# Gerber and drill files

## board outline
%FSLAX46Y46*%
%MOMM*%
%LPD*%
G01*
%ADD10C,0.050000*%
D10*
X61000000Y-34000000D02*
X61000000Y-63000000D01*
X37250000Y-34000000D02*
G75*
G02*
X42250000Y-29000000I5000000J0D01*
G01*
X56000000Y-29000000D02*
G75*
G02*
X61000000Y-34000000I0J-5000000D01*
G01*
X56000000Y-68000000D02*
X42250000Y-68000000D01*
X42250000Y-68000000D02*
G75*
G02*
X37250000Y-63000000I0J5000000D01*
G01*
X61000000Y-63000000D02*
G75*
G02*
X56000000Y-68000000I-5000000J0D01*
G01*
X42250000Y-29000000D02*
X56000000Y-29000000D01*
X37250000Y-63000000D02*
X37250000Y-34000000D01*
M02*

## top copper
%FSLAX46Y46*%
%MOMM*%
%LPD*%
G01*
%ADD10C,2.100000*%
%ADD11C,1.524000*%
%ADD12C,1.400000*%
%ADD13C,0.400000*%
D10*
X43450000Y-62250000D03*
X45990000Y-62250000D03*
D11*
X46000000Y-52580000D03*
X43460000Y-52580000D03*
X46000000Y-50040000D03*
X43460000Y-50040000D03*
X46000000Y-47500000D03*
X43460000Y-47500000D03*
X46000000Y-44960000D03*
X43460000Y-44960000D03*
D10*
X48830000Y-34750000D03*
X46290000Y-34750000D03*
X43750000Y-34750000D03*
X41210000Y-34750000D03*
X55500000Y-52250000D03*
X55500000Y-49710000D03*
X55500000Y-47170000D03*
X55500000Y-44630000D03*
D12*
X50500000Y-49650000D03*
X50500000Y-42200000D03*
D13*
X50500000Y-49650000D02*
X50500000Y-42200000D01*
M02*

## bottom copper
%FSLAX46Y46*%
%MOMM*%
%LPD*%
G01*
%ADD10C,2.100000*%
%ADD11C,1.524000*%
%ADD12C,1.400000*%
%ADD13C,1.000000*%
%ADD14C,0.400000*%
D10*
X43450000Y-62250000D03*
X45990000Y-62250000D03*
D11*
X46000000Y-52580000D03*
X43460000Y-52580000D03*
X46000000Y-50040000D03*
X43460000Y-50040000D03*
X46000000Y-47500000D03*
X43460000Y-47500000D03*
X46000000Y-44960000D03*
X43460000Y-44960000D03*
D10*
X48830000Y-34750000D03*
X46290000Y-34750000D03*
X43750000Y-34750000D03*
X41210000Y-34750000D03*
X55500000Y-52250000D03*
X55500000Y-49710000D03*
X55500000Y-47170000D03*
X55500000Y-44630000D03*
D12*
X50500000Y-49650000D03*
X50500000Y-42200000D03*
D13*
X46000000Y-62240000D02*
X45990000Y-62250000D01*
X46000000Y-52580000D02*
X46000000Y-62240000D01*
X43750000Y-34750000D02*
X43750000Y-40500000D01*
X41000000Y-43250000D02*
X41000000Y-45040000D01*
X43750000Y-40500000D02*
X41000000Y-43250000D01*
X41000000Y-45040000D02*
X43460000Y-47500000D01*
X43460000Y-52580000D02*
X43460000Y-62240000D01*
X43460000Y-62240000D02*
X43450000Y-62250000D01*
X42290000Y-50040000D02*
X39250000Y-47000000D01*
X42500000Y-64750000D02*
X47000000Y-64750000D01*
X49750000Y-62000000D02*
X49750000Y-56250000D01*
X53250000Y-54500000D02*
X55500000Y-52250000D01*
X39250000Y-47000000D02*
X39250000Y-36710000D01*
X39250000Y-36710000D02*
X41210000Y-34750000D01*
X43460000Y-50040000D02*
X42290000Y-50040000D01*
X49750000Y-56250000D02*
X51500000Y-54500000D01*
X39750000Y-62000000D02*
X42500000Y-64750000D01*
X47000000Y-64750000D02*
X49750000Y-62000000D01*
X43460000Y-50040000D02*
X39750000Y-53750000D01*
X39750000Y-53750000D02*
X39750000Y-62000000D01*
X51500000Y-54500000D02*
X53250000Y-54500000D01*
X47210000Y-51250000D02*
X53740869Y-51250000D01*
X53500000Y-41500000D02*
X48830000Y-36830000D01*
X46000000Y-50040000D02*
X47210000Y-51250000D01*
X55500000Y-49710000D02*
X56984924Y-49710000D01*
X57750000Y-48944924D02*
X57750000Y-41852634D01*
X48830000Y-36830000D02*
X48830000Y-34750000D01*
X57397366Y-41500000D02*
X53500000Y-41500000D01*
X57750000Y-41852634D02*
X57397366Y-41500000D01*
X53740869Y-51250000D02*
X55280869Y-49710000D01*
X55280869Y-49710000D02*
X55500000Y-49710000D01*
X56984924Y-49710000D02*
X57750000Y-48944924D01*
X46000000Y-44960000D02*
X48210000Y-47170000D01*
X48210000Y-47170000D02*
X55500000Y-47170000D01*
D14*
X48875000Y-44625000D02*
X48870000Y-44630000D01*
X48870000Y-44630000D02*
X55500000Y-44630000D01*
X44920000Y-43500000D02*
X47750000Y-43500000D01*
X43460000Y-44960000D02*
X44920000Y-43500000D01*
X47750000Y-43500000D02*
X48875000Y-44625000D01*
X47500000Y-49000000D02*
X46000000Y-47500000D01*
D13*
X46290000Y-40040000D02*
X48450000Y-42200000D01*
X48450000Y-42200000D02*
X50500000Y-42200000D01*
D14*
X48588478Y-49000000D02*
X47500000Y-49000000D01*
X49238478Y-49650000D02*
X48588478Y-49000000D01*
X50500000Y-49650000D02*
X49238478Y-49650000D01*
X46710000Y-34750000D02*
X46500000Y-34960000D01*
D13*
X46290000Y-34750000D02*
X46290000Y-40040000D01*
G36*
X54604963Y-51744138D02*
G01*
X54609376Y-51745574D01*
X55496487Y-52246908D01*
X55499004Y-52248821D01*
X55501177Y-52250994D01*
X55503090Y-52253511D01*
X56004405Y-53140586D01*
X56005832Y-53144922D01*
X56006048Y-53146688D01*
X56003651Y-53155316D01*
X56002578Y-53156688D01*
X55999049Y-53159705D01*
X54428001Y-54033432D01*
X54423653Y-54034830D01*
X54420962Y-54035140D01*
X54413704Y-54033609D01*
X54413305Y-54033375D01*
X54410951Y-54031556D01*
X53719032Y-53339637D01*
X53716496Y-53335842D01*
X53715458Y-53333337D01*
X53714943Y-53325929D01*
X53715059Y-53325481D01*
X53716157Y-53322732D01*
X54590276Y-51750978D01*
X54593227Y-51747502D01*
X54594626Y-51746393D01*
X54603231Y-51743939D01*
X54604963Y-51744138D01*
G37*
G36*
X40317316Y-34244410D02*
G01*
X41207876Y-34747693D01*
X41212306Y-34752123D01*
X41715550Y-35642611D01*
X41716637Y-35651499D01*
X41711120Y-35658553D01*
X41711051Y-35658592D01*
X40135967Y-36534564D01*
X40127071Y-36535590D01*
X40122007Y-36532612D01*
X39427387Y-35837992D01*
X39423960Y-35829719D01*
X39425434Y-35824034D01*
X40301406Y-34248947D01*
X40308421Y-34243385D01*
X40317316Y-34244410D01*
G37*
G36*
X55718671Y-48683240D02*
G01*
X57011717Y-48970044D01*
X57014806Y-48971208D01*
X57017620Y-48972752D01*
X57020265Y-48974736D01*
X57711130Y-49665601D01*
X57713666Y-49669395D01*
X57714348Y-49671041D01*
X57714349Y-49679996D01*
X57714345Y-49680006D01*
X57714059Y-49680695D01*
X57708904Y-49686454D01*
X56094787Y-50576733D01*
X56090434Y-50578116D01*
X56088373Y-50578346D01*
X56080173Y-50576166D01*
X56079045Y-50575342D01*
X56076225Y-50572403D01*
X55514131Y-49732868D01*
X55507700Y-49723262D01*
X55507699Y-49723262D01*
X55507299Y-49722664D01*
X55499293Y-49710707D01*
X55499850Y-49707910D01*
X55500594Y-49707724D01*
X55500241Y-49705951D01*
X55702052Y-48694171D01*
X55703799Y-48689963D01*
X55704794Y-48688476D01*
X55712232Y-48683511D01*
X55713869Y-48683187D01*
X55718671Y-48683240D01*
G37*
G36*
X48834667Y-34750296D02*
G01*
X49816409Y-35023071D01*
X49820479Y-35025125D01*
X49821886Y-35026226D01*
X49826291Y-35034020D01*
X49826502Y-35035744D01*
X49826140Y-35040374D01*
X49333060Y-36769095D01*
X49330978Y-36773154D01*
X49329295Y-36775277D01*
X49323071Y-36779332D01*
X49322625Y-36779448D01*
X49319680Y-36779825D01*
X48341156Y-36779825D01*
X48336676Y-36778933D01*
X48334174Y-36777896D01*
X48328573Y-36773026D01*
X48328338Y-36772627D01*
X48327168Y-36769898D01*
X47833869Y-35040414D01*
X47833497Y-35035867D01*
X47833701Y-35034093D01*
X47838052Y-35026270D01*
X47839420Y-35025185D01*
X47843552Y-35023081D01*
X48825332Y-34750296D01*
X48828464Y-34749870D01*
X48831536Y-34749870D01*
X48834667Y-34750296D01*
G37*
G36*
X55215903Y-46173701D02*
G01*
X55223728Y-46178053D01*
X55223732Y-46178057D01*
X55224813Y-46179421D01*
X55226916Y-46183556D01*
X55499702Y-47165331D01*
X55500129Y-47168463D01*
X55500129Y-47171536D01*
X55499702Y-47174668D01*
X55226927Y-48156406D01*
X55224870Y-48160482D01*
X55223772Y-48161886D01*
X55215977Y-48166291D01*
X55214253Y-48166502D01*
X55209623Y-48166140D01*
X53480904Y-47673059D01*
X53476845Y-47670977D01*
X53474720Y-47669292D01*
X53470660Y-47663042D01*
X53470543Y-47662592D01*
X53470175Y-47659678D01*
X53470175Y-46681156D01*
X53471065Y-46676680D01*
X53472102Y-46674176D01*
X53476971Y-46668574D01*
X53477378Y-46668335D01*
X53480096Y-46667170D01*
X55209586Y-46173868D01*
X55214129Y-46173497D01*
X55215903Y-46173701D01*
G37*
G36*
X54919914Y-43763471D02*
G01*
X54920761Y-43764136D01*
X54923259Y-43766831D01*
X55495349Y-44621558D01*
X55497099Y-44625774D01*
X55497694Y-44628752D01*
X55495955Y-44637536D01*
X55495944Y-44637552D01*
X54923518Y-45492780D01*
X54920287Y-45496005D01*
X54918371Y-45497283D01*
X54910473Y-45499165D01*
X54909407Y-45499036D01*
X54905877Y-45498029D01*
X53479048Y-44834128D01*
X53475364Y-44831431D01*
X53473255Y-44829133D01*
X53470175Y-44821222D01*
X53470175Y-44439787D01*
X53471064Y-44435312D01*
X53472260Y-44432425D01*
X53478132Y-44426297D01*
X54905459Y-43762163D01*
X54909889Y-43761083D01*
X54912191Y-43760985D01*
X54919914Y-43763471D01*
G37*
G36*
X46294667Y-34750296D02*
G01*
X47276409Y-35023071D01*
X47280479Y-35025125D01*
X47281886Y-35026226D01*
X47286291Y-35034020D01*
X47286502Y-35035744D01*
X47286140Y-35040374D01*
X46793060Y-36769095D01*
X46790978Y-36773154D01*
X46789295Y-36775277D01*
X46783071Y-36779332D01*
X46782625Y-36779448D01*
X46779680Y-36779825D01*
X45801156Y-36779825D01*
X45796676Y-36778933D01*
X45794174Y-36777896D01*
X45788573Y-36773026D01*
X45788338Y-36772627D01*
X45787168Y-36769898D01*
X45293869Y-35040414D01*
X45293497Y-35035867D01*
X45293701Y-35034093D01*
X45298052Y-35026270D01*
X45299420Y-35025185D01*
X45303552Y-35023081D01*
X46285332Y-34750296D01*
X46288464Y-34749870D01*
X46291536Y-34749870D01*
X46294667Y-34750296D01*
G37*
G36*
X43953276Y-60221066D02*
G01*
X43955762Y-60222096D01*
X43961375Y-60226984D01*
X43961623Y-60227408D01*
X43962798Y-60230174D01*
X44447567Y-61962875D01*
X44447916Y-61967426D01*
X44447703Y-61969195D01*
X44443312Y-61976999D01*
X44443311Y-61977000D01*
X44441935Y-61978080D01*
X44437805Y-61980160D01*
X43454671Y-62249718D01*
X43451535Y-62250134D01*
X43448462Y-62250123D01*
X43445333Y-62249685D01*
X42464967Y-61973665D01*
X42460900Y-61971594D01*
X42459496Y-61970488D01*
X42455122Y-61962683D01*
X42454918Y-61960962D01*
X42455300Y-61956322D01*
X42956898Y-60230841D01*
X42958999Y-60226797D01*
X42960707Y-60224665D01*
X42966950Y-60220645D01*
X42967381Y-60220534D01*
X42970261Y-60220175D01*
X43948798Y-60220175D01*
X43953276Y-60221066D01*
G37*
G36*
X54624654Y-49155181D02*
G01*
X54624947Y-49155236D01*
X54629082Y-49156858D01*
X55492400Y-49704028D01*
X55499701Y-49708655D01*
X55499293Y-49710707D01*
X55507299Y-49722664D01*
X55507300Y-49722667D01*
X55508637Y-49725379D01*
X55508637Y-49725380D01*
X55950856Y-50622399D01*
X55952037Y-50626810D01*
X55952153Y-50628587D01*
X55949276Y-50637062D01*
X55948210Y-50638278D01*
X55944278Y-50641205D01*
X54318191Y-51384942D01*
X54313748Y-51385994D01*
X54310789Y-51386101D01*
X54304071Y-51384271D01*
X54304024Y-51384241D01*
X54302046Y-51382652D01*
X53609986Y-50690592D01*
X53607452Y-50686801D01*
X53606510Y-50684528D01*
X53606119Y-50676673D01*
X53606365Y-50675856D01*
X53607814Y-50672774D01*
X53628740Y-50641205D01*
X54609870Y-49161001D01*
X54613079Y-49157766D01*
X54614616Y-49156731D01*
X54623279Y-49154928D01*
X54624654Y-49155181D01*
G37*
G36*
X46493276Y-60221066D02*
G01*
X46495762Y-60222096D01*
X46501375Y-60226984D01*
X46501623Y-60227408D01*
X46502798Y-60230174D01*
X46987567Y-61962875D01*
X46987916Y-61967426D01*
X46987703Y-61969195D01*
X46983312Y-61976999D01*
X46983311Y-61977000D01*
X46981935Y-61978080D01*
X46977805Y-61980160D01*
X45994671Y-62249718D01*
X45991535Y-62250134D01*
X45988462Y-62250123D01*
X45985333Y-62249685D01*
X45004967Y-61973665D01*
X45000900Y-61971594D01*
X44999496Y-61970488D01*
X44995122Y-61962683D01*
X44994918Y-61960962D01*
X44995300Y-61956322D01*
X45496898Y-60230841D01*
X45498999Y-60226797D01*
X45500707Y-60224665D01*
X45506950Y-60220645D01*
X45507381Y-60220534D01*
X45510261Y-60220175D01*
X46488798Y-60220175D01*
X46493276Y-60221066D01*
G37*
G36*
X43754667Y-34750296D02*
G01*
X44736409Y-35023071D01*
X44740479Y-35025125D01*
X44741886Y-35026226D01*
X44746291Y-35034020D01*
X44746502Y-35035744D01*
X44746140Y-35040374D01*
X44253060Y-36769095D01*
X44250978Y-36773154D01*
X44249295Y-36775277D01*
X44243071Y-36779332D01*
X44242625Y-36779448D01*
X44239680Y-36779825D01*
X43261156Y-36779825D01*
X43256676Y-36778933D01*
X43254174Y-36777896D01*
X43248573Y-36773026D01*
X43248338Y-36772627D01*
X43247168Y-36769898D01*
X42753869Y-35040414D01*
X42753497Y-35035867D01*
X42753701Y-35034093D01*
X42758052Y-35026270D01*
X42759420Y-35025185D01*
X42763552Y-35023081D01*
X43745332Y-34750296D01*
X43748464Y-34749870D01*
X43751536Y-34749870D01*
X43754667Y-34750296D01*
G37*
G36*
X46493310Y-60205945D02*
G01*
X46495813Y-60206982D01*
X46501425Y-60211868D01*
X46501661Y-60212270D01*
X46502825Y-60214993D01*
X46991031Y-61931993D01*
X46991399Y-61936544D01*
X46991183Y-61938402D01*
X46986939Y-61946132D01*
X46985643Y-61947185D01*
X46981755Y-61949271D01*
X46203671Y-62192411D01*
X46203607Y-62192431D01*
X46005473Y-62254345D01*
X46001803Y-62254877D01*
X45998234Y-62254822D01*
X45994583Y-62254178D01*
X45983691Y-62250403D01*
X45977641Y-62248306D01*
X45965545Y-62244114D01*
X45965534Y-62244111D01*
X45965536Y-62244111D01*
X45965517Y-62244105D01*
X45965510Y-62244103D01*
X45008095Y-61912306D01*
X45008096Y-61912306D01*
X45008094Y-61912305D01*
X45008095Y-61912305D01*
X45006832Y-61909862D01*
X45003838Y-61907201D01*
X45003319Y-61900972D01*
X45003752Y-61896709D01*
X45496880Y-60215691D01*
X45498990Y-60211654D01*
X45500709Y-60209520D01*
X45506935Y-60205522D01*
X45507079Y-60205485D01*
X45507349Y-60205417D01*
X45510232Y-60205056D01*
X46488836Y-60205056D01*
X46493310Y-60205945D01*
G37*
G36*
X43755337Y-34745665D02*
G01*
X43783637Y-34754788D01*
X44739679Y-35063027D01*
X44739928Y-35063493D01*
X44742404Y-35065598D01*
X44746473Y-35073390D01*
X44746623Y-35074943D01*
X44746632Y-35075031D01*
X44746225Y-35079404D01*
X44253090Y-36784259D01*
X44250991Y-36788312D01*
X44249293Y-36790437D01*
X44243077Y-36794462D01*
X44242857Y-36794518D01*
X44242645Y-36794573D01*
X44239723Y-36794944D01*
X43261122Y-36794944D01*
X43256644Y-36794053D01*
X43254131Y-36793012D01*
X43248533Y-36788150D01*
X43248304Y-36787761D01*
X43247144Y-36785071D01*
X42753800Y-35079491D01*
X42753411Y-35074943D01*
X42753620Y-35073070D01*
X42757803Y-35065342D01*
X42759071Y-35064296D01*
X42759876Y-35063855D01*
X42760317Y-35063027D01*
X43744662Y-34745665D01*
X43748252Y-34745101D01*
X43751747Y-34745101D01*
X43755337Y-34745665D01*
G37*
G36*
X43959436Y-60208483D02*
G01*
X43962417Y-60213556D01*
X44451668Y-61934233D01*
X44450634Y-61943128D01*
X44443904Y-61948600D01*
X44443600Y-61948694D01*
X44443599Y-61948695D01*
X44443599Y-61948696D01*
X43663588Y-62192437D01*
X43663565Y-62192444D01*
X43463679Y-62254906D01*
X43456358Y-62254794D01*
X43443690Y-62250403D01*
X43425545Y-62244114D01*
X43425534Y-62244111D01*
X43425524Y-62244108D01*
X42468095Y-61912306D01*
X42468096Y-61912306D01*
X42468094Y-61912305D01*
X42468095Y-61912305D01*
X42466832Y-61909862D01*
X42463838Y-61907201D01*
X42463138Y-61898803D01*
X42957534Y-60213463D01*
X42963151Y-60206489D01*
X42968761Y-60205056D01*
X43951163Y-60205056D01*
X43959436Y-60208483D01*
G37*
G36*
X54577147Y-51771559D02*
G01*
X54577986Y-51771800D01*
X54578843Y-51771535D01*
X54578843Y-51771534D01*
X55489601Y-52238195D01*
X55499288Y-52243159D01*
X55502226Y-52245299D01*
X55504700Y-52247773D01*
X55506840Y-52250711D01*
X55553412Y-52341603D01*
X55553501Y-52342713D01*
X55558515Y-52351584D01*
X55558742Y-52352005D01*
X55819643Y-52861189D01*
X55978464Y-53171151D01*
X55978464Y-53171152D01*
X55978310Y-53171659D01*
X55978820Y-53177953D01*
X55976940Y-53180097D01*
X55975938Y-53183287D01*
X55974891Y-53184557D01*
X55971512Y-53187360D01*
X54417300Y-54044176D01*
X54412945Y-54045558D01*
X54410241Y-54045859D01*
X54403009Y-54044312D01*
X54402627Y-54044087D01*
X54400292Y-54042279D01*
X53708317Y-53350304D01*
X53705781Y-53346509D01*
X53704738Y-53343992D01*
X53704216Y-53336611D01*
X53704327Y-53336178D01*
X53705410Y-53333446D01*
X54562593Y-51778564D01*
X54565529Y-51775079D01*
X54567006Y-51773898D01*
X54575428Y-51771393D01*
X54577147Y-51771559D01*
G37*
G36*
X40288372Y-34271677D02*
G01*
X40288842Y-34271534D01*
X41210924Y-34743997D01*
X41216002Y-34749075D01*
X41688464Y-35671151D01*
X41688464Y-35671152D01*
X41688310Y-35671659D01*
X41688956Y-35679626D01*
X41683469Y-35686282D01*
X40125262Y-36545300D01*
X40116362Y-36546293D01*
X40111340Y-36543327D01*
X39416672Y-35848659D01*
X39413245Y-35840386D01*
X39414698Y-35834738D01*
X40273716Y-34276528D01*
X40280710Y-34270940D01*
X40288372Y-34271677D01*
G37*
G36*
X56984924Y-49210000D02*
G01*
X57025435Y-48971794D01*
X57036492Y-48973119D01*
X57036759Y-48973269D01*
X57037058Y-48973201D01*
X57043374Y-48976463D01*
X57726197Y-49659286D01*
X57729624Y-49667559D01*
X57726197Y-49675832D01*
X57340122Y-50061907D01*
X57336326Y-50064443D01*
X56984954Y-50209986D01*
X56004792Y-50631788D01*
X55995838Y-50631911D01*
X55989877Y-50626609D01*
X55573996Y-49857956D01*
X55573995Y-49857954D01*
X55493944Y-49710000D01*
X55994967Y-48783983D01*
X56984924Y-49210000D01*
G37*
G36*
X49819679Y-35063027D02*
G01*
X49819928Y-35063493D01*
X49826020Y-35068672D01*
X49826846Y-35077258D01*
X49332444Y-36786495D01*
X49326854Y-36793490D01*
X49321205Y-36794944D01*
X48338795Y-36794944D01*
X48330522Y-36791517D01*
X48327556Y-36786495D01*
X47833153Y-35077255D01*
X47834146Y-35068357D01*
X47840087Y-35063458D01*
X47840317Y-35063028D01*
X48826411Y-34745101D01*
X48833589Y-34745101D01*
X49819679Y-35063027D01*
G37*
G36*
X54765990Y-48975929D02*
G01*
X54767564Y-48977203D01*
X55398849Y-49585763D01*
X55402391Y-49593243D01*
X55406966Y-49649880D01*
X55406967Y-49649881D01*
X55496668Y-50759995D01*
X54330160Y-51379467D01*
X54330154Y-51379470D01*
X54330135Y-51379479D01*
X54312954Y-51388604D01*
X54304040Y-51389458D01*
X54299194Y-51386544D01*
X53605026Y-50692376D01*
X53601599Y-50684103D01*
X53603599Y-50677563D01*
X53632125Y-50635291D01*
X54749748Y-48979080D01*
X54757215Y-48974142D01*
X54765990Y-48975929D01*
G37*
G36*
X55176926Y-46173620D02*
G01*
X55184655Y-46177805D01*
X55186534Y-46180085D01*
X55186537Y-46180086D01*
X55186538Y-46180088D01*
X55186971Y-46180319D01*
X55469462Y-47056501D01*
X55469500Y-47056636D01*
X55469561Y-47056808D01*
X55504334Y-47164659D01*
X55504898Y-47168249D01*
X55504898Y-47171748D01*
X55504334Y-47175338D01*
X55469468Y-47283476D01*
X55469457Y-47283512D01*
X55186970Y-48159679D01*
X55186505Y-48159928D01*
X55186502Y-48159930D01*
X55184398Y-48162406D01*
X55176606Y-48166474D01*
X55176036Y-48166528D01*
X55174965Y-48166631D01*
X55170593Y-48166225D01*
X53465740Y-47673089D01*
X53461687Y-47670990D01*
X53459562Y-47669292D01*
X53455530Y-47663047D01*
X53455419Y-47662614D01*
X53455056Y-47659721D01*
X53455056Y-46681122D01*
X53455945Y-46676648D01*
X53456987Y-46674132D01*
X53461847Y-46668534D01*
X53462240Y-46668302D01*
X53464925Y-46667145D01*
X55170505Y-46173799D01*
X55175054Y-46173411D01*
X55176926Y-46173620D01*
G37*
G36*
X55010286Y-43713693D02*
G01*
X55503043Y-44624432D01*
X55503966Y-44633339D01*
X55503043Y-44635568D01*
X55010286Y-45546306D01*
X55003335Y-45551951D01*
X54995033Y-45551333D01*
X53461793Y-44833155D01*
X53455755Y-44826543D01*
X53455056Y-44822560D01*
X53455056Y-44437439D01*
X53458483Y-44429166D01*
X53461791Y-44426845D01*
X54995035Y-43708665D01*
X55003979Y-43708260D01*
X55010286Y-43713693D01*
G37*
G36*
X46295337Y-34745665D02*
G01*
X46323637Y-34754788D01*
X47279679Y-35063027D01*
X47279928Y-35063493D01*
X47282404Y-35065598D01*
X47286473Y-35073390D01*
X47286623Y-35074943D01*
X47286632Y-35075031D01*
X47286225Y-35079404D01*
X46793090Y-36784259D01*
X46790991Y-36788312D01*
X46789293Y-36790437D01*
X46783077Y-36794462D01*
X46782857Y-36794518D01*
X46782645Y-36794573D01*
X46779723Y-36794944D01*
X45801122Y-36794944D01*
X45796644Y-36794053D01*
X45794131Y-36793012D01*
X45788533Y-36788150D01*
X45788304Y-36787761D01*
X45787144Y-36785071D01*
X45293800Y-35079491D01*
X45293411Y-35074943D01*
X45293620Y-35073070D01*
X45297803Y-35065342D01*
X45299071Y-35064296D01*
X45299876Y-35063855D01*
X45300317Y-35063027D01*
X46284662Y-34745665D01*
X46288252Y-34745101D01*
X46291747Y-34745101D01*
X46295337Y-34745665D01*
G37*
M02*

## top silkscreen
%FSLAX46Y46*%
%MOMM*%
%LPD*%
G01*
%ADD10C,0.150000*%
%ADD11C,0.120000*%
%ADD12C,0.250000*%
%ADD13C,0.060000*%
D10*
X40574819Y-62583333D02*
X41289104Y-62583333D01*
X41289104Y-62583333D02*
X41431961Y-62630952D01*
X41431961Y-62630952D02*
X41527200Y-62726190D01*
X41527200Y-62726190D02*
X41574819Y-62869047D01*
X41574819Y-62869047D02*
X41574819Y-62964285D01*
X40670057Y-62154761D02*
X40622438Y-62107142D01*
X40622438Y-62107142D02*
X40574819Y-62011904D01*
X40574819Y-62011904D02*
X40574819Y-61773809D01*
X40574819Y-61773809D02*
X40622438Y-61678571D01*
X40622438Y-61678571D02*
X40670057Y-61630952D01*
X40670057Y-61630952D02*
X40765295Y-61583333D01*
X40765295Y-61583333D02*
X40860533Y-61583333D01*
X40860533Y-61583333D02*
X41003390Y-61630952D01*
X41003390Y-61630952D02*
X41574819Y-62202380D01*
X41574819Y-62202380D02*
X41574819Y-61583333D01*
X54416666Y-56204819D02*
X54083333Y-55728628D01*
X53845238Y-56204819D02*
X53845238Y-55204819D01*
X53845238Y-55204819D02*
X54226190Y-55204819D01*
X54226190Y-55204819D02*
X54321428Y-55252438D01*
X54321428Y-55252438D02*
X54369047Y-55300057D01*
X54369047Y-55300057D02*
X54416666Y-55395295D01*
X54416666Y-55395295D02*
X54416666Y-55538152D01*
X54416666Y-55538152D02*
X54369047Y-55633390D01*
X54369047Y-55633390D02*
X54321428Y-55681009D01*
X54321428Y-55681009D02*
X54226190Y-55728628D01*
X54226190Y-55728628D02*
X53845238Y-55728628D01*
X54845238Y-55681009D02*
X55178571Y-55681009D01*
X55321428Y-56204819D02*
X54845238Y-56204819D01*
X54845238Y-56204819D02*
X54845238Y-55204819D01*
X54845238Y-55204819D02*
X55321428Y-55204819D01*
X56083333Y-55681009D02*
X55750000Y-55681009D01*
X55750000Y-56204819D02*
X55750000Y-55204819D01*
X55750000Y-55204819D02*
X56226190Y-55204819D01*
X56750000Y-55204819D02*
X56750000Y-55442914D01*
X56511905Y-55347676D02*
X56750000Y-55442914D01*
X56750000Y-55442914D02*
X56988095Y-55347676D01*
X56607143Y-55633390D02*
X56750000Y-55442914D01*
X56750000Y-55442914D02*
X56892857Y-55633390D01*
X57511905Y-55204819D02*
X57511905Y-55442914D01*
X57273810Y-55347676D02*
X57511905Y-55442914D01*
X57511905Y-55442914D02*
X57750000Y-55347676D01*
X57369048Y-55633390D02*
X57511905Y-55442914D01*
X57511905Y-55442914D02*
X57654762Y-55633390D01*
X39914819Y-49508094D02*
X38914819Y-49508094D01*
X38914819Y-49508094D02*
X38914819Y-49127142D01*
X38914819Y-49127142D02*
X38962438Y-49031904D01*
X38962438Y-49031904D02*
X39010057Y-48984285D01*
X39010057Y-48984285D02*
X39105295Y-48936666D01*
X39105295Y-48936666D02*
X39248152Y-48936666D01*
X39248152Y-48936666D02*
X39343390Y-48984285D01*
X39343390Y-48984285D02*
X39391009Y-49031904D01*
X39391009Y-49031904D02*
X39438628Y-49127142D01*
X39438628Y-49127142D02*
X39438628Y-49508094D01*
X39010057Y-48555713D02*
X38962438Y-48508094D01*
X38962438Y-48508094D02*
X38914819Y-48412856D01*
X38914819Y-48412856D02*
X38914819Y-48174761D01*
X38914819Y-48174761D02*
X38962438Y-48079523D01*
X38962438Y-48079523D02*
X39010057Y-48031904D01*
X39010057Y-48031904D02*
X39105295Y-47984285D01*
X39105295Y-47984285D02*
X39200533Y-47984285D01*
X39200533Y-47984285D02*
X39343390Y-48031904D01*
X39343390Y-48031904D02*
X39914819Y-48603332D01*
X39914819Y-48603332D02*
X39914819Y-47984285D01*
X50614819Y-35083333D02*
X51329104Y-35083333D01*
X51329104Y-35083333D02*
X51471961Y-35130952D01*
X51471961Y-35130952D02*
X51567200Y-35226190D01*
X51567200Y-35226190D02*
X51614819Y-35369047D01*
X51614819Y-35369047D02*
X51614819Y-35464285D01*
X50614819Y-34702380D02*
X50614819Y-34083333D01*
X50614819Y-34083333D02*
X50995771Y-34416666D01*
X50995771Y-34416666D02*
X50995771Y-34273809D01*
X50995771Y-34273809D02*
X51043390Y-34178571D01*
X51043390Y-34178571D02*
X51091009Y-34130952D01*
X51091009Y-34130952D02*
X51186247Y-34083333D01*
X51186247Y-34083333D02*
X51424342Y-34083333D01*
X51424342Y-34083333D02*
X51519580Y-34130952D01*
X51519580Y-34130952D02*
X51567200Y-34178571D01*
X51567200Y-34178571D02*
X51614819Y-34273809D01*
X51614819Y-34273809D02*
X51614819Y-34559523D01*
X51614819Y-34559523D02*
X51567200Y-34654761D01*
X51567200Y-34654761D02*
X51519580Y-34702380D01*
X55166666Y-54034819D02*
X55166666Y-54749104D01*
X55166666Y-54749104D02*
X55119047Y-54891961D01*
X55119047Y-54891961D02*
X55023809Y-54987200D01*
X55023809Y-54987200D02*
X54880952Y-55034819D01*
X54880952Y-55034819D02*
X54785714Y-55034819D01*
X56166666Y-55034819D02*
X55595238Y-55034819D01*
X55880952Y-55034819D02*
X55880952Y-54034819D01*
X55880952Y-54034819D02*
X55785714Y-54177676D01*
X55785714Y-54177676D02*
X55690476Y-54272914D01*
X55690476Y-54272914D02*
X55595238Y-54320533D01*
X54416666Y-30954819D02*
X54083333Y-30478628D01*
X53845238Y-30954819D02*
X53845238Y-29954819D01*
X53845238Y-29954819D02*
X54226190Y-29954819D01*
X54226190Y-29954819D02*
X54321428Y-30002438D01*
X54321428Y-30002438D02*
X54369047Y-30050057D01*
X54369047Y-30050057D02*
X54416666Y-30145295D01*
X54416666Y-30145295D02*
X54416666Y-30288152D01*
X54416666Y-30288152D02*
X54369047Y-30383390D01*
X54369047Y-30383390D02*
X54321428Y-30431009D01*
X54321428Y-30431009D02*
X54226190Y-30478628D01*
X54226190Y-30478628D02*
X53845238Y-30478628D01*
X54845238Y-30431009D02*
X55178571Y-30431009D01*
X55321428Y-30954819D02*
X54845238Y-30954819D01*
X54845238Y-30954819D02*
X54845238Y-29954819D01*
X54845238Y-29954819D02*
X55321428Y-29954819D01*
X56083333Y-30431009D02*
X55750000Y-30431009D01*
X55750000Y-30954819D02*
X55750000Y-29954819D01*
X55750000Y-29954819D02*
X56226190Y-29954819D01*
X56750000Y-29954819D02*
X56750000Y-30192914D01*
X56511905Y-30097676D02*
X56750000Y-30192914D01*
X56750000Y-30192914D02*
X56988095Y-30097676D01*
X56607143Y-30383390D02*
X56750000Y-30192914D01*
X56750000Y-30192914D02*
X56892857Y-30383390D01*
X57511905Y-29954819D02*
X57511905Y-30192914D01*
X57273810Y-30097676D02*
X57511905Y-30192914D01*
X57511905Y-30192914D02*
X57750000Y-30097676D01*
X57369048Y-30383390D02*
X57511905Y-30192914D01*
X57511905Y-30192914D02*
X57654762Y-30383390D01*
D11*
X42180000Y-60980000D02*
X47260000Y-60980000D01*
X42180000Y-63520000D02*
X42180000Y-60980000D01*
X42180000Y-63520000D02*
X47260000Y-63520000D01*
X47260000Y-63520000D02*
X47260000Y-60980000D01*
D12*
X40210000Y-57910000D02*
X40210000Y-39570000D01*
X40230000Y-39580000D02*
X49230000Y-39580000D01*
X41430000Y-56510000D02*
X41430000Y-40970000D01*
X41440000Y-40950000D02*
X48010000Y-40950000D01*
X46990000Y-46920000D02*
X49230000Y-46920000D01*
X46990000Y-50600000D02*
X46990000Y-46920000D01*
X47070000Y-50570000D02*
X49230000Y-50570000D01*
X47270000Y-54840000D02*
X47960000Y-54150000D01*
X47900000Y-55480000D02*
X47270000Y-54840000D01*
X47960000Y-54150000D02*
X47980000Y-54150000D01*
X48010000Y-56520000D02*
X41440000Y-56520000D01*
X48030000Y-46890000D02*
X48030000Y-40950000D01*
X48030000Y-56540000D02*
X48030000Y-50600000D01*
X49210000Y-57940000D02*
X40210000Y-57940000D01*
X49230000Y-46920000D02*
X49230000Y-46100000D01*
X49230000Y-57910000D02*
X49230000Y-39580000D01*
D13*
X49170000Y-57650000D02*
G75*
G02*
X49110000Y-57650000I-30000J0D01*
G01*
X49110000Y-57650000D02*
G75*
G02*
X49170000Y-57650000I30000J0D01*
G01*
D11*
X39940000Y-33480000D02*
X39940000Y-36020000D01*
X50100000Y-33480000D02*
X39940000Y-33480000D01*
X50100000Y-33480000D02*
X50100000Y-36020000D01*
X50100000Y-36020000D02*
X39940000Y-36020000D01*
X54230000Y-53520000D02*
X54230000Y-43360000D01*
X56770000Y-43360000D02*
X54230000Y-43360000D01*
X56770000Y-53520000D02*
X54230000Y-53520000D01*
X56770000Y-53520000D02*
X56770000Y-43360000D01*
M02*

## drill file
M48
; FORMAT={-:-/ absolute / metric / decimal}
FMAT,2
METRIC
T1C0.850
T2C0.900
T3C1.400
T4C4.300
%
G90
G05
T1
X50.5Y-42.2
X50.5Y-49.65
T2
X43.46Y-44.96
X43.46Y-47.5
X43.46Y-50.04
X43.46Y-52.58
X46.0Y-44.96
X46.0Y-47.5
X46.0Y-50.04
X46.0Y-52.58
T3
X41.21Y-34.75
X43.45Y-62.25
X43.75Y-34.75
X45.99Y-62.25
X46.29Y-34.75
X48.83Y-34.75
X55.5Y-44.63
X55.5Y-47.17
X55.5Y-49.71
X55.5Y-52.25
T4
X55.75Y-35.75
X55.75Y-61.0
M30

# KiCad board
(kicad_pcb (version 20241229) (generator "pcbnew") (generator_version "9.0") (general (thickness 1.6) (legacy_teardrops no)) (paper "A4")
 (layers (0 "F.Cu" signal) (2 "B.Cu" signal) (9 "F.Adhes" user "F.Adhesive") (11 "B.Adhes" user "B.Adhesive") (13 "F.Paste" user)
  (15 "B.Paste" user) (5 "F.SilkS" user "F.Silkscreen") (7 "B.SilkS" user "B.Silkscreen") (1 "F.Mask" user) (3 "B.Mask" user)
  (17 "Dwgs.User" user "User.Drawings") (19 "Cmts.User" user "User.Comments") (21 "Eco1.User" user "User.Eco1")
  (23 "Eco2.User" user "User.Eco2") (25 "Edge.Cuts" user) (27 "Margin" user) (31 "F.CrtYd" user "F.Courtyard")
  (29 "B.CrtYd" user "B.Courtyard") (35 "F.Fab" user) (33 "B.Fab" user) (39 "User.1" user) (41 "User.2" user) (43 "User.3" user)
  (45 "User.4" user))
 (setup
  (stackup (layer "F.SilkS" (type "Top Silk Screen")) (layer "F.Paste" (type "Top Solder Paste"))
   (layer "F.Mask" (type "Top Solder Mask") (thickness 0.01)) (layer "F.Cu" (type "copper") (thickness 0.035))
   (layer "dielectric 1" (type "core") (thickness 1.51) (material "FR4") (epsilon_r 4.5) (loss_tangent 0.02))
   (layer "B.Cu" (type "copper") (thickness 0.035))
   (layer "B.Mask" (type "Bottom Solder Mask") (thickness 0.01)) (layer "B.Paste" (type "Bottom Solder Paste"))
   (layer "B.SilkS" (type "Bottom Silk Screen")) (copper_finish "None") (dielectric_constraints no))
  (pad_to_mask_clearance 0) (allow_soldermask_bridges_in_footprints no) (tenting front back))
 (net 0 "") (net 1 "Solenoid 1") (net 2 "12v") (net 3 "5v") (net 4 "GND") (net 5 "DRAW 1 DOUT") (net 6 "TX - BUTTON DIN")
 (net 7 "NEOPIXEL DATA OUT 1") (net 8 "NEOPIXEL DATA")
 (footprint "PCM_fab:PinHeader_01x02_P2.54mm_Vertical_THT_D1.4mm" (layer "F.Cu") (at 43.45 62.25 90)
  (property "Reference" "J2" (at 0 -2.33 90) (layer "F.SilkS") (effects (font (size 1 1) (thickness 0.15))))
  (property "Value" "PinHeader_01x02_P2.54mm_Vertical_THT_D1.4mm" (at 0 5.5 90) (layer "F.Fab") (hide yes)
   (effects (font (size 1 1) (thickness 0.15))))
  (fp_line (start 1.27 -1.27) (end 1.27 3.81) (stroke (width 0.12) (type solid)) (layer "F.SilkS"))
  (fp_line (start -1.27 -1.27) (end 1.27 -1.27) (stroke (width 0.12) (type solid)) (layer "F.SilkS"))
  (fp_line (start -1.27 -1.27) (end -1.27 3.81) (stroke (width 0.12) (type solid)) (layer "F.SilkS"))
  (fp_line (start -1.27 3.81) (end 1.27 3.81) (stroke (width 0.12) (type solid)) (layer "F.SilkS"))
  (pad "1" thru_hole circle (at 0 0 90) (size 2.1 2.1) (drill 1.4) (layers "*.Cu" "*.Mask") (remove_unused_layers no) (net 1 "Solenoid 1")
   (teardrops (best_length_ratio 0.5) (max_length 1) (best_width_ratio 1) (max_width 2) (curved_edges no) (filter_ratio 0.9) (enabled yes)
    (allow_two_segments yes) (prefer_zone_connections yes)))
  (pad "2" thru_hole circle (at 0 2.54 90) (size 2.1 2.1) (drill 1.4) (layers "*.Cu" "*.Mask") (remove_unused_layers no) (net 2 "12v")
   (teardrops (best_length_ratio 0.5) (max_length 1) (best_width_ratio 1) (max_width 2) (curved_edges no) (filter_ratio 0.9) (enabled yes)
    (allow_two_segments yes) (prefer_zone_connections yes))))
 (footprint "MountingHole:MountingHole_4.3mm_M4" (layer "F.Cu") (at 55.75 61)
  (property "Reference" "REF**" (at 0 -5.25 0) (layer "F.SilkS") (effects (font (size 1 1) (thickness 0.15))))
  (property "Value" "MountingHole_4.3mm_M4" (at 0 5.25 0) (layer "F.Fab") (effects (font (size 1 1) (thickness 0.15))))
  (pad "" np_thru_hole circle (at 0 0) (size 4.3 4.3) (drill 4.3) (layers "*.Cu" "*.Mask")))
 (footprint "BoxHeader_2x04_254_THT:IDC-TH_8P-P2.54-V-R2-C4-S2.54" (layer "F.Cu") (at 44.73 48.77 90)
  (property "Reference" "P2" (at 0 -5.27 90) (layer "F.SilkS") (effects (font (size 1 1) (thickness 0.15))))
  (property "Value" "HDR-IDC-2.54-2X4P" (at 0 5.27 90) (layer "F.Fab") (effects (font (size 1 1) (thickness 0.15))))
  (fp_line (start -9.14 -4.52) (end 9.2 -4.52) (stroke (width 0.25) (type solid)) (layer "F.SilkS"))
  (fp_line (start 9.19 -4.5) (end 9.19 4.5) (stroke (width 0.25) (type solid)) (layer "F.SilkS"))
  (fp_line (start -7.74 -3.3) (end 7.8 -3.3) (stroke (width 0.25) (type solid)) (layer "F.SilkS"))
  (fp_line (start 7.82 -3.29) (end 7.82 3.28) (stroke (width 0.25) (type solid)) (layer "F.SilkS"))
  (fp_line (start 1.85 2.26) (end 1.85 4.5) (stroke (width 0.25) (type solid)) (layer "F.SilkS"))
  (fp_line (start -1.83 2.26) (end 1.85 2.26) (stroke (width 0.25) (type solid)) (layer "F.SilkS"))
  (fp_line (start -1.8 2.34) (end -1.8 4.5) (stroke (width 0.25) (type solid)) (layer "F.SilkS"))
  (fp_line (start -6.07 2.54) (end -5.38 3.23) (stroke (width 0.25) (type solid)) (layer "F.SilkS"))
  (fp_line (start -6.71 3.17) (end -6.07 2.54) (stroke (width 0.25) (type solid)) (layer "F.SilkS"))
  (fp_line (start -5.38 3.23) (end -5.38 3.25) (stroke (width 0.25) (type solid)) (layer "F.SilkS"))
  (fp_line (start -7.75 3.28) (end -7.75 -3.29) (stroke (width 0.25) (type solid)) (layer "F.SilkS"))
  (fp_line (start 1.88 3.3) (end 7.82 3.3) (stroke (width 0.25) (type solid)) (layer "F.SilkS"))
  (fp_line (start -7.77 3.3) (end -1.83 3.3) (stroke (width 0.25) (type solid)) (layer "F.SilkS"))
  (fp_line (start -9.17 4.48) (end -9.17 -4.52) (stroke (width 0.25) (type solid)) (layer "F.SilkS"))
  (fp_line (start 1.85 4.5) (end 2.67 4.5) (stroke (width 0.25) (type solid)) (layer "F.SilkS"))
  (fp_line (start -9.14 4.5) (end 9.19 4.5) (stroke (width 0.25) (type solid)) (layer "F.SilkS"))
  (fp_circle (center -8.88 4.41) (end -8.85 4.41) (stroke (width 0.06) (type solid)) (fill no) (layer "F.SilkS"))
  (pad "1" thru_hole circle (at -3.81 1.27 90) (size 1.524 1.524) (drill 0.9) (layers "*.Cu" "*.Mask") (remove_unused_layers no)
   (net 2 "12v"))
  (pad "2" thru_hole circle (at -3.81 -1.27 90) (size 1.524 1.524) (drill 0.9) (layers "*.Cu" "*.Mask") (remove_unused_layers no)
   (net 1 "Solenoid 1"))
  (pad "3" thru_hole circle (at -1.27 1.27 90) (size 1.524 1.524) (drill 0.9) (layers "*.Cu" "*.Mask") (remove_unused_layers no)
   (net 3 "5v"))
  (pad "4" thru_hole circle (at -1.27 -1.27 90) (size 1.524 1.524) (drill 0.9) (layers "*.Cu" "*.Mask") (remove_unused_layers no)
   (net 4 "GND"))
  (pad "5" thru_hole circle (at 1.27 1.27 90) (size 1.524 1.524) (drill 0.9) (layers "*.Cu" "*.Mask") (remove_unused_layers no)
   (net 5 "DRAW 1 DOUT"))
  (pad "6" thru_hole circle (at 1.27 -1.27 90) (size 1.524 1.524) (drill 0.9) (layers "*.Cu" "*.Mask") (remove_unused_layers no)
   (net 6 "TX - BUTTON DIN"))
  (pad "7" thru_hole circle (at 3.81 1.27 90) (size 1.524 1.524) (drill 0.9) (layers "*.Cu" "*.Mask") (remove_unused_layers no)
   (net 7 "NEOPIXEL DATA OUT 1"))
  (pad "8" thru_hole circle (at 3.81 -1.27 90) (size 1.524 1.524) (drill 0.9) (layers "*.Cu" "*.Mask") (remove_unused_layers no)
   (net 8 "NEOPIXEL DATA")))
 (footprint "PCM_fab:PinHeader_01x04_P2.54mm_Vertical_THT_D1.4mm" (layer "F.Cu") (at 48.83 34.75 -90)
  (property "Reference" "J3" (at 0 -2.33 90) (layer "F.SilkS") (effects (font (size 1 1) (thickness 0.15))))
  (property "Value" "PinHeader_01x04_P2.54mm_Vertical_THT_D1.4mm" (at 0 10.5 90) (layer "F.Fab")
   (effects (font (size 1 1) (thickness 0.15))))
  (fp_line (start -1.27 8.89) (end 1.27 8.89) (stroke (width 0.12) (type solid)) (layer "F.SilkS"))
  (fp_line (start -1.27 -1.27) (end -1.27 8.89) (stroke (width 0.12) (type solid)) (layer "F.SilkS"))
  (fp_line (start -1.27 -1.27) (end 1.27 -1.27) (stroke (width 0.12) (type solid)) (layer "F.SilkS"))
  (fp_line (start 1.27 -1.27) (end 1.27 8.89) (stroke (width 0.12) (type solid)) (layer "F.SilkS"))
  (pad "1" thru_hole circle (at 0 0 270) (size 2.1 2.1) (drill 1.4) (layers "*.Cu" "*.Mask") (remove_unused_layers no) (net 3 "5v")
   (teardrops (best_length_ratio 0.5) (max_length 1) (best_width_ratio 1) (max_width 2) (curved_edges no) (filter_ratio 0.9) (enabled yes)
    (allow_two_segments yes) (prefer_zone_connections yes)))
  (pad "2" thru_hole circle (at 0 2.54 270) (size 2.1 2.1) (drill 1.4) (layers "*.Cu" "*.Mask") (remove_unused_layers no)
   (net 5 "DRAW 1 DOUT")
   (teardrops (best_length_ratio 0.5) (max_length 1) (best_width_ratio 1) (max_width 2) (curved_edges no) (filter_ratio 0.9) (enabled yes)
    (allow_two_segments yes) (prefer_zone_connections yes)))
  (pad "3" thru_hole circle (at 0 5.08 270) (size 2.1 2.1) (drill 1.4) (layers "*.Cu" "*.Mask") (remove_unused_layers no)
   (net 6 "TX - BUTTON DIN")
   (teardrops (best_length_ratio 0.5) (max_length 1) (best_width_ratio 1) (max_width 2) (curved_edges no) (filter_ratio 0.9) (enabled yes)
    (allow_two_segments yes) (prefer_zone_connections yes)))
  (pad "4" thru_hole circle (at 0 7.62 270) (size 2.1 2.1) (drill 1.4) (layers "*.Cu" "*.Mask") (remove_unused_layers no) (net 4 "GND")
   (teardrops (best_length_ratio 0.5) (max_length 1) (best_width_ratio 1) (max_width 2) (curved_edges no) (filter_ratio 0.9) (enabled yes)
    (allow_two_segments yes) (prefer_zone_connections yes))))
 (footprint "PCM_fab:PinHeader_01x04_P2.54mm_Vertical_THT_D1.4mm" (layer "F.Cu") (at 55.5 52.25 180)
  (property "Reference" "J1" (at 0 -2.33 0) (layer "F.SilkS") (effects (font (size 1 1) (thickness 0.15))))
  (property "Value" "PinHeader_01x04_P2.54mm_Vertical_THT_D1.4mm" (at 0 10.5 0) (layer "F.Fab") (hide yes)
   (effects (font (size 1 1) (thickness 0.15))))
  (fp_line (start 1.27 -1.27) (end 1.27 8.89) (stroke (width 0.12) (type solid)) (layer "F.SilkS"))
  (fp_line (start -1.27 8.89) (end 1.27 8.89) (stroke (width 0.12) (type solid)) (layer "F.SilkS"))
  (fp_line (start -1.27 -1.27) (end 1.27 -1.27) (stroke (width 0.12) (type solid)) (layer "F.SilkS"))
  (fp_line (start -1.27 -1.27) (end -1.27 8.89) (stroke (width 0.12) (type solid)) (layer "F.SilkS"))
  (pad "1" thru_hole circle (at 0 0 180) (size 2.1 2.1) (drill 1.4) (layers "*.Cu" "*.Mask") (remove_unused_layers no) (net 4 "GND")
   (teardrops (best_length_ratio 0.5) (max_length 1) (best_width_ratio 1) (max_width 2) (curved_edges no) (filter_ratio 0.9) (enabled yes)
    (allow_two_segments yes) (prefer_zone_connections yes)))
  (pad "2" thru_hole circle (at 0 2.54 180) (size 2.1 2.1) (drill 1.4) (layers "*.Cu" "*.Mask") (remove_unused_layers no) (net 3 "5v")
   (teardrops (best_length_ratio 0.5) (max_length 1) (best_width_ratio 1) (max_width 2) (curved_edges no) (filter_ratio 0.9) (enabled yes)
    (allow_two_segments yes) (prefer_zone_connections yes)))
  (pad "3" thru_hole circle (at 0 5.08 180) (size 2.1 2.1) (drill 1.4) (layers "*.Cu" "*.Mask") (remove_unused_layers no)
   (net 7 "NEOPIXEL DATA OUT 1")
   (teardrops (best_length_ratio 0.5) (max_length 1) (best_width_ratio 1) (max_width 2) (curved_edges no) (filter_ratio 0.9) (enabled yes)
    (allow_two_segments yes) (prefer_zone_connections yes)))
  (pad "4" thru_hole circle (at 0 7.62 180) (size 2.1 2.1) (drill 1.4) (layers "*.Cu" "*.Mask") (remove_unused_layers no)
   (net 8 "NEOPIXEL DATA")
   (teardrops (best_length_ratio 0.5) (max_length 1) (best_width_ratio 1) (max_width 2) (curved_edges no) (filter_ratio 0.9) (enabled yes)
    (allow_two_segments yes) (prefer_zone_connections yes))))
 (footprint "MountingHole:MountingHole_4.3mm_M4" (layer "F.Cu") (at 55.75 35.75)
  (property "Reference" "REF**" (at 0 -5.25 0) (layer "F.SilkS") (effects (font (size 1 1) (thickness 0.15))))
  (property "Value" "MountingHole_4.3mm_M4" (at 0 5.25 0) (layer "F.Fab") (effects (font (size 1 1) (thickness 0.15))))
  (pad "" np_thru_hole circle (at 0 0) (size 4.3 4.3) (drill 4.3) (layers "*.Cu" "*.Mask")))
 (gr_line (start 61 34) (end 61 63) (stroke (width 0.05) (type default)) (layer "Edge.Cuts"))
 (gr_arc (start 37.25 34) (mid 38.714466 30.464466) (end 42.25 29) (stroke (width 0.05) (type default)) (layer "Edge.Cuts"))
 (gr_arc (start 56 29) (mid 59.535534 30.464466) (end 61 34) (stroke (width 0.05) (type default)) (layer "Edge.Cuts"))
 (gr_line (start 56 68) (end 42.25 68) (stroke (width 0.05) (type default)) (layer "Edge.Cuts"))
 (gr_arc (start 42.25 68) (mid 38.714466 66.535534) (end 37.25 63) (stroke (width 0.05) (type default)) (layer "Edge.Cuts"))
 (gr_arc (start 61 63) (mid 59.535534 66.535534) (end 56 68) (stroke (width 0.05) (type default)) (layer "Edge.Cuts"))
 (gr_line (start 42.25 29) (end 56 29) (stroke (width 0.05) (type default)) (layer "Edge.Cuts"))
 (gr_line (start 37.25 63) (end 37.25 34) (stroke (width 0.05) (type default)) (layer "Edge.Cuts"))
 (segment (start 46 62.24) (end 45.99 62.25) (width 1) (layer "B.Cu") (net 2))
 (segment (start 46 52.58) (end 46 62.24) (width 1) (layer "B.Cu") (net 2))
 (segment (start 43.75 34.75) (end 43.75 40.5) (width 1) (layer "B.Cu") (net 6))
 (segment (start 41 43.25) (end 41 45.04) (width 1) (layer "B.Cu") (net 6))
 (segment (start 43.75 40.5) (end 41 43.25) (width 1) (layer "B.Cu") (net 6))
 (segment (start 41 45.04) (end 43.46 47.5) (width 1) (layer "B.Cu") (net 6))
 (segment (start 43.46 52.58) (end 43.46 62.24) (width 1) (layer "B.Cu") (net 1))
 (segment (start 43.46 62.24) (end 43.45 62.25) (width 1) (layer "B.Cu") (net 1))
 (segment (start 42.29 50.04) (end 39.25 47) (width 1) (layer "B.Cu") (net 4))
 (segment (start 42.5 64.75) (end 47 64.75) (width 1) (layer "B.Cu") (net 4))
 (segment (start 49.75 62) (end 49.75 56.25) (width 1) (layer "B.Cu") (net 4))
 (segment (start 53.25 54.5) (end 55.5 52.25) (width 1) (layer "B.Cu") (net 4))
 (segment (start 39.25 47) (end 39.25 36.71) (width 1) (layer "B.Cu") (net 4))
 (segment (start 39.25 36.71) (end 41.21 34.75) (width 1) (layer "B.Cu") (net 4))
 (segment (start 43.46 50.04) (end 42.29 50.04) (width 1) (layer "B.Cu") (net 4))
 (segment (start 49.75 56.25) (end 51.5 54.5) (width 1) (layer "B.Cu") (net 4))
 (segment (start 39.75 62) (end 42.5 64.75) (width 1) (layer "B.Cu") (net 4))
 (segment (start 47 64.75) (end 49.75 62) (width 1) (layer "B.Cu") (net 4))
 (segment (start 43.46 50.04) (end 39.75 53.75) (width 1) (layer "B.Cu") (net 4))
 (segment (start 39.75 53.75) (end 39.75 62) (width 1) (layer "B.Cu") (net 4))
 (segment (start 51.5 54.5) (end 53.25 54.5) (width 1) (layer "B.Cu") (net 4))
 (segment (start 47.21 51.25) (end 53.740869 51.25) (width 1) (layer "B.Cu") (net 3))
 (segment (start 53.5 41.5) (end 48.83 36.83) (width 1) (layer "B.Cu") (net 3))
 (segment (start 46 50.04) (end 47.21 51.25) (width 1) (layer "B.Cu") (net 3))
 (segment (start 55.5 49.71) (end 56.984924 49.71) (width 1) (layer "B.Cu") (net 3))
 (segment (start 57.75 48.944924) (end 57.75 41.852634) (width 1) (layer "B.Cu") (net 3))
 (segment (start 48.83 36.83) (end 48.83 34.75) (width 1) (layer "B.Cu") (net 3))
 (segment (start 57.397366 41.5) (end 53.5 41.5) (width 1) (layer "B.Cu") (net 3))
 (segment (start 57.75 41.852634) (end 57.397366 41.5) (width 1) (layer "B.Cu") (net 3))
 (segment (start 53.740869 51.25) (end 55.280869 49.71) (width 1) (layer "B.Cu") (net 3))
 (segment (start 55.280869 49.71) (end 55.5 49.71) (width 1) (layer "B.Cu") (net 3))
 (segment (start 56.984924 49.71) (end 57.75 48.944924) (width 1) (layer "B.Cu") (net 3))
 (segment (start 46 44.96) (end 48.21 47.17) (width 1) (layer "B.Cu") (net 7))
 (segment (start 48.21 47.17) (end 55.5 47.17) (width 1) (layer "B.Cu") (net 7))
 (segment (start 48.875 44.625) (end 48.87 44.63) (width 0.4) (layer "B.Cu") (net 8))
 (segment (start 48.87 44.63) (end 55.5 44.63) (width 0.4) (layer "B.Cu") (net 8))
 (segment (start 44.92 43.5) (end 47.75 43.5) (width 0.4) (layer "B.Cu") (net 8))
 (segment (start 43.46 44.96) (end 44.92 43.5) (width 0.4) (layer "B.Cu") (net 8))
 (segment (start 47.75 43.5) (end 48.875 44.625) (width 0.4) (layer "B.Cu") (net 8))
 (segment (start 50.5 49.65) (end 50.5 42.2) (width 0.4) (layer "F.Cu") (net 5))
 (via (at 50.5 49.65) (size 1.4) (drill 0.85) (layers "F.Cu" "B.Cu") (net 5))
 (via (at 50.5 42.2) (size 1.4) (drill 0.85) (layers "F.Cu" "B.Cu") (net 5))
 (segment (start 47.5 49) (end 46 47.5) (width 0.4) (layer "B.Cu") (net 5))
 (segment (start 46.29 40.04) (end 48.45 42.2) (width 1) (layer "B.Cu") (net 5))
 (segment (start 48.45 42.2) (end 50.5 42.2) (width 1) (layer "B.Cu") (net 5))
 (segment (start 48.588478 49) (end 47.5 49) (width 0.4) (layer "B.Cu") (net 5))
 (segment (start 49.238478 49.65) (end 48.588478 49) (width 0.4) (layer "B.Cu") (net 5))
 (segment (start 50.5 49.65) (end 49.238478 49.65) (width 0.4) (layer "B.Cu") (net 5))
 (segment (start 46.71 34.75) (end 46.5 34.96) (width 0.4) (layer "B.Cu") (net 5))
 (segment (start 46.29 34.75) (end 46.29 40.04) (width 1) (layer "B.Cu") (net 5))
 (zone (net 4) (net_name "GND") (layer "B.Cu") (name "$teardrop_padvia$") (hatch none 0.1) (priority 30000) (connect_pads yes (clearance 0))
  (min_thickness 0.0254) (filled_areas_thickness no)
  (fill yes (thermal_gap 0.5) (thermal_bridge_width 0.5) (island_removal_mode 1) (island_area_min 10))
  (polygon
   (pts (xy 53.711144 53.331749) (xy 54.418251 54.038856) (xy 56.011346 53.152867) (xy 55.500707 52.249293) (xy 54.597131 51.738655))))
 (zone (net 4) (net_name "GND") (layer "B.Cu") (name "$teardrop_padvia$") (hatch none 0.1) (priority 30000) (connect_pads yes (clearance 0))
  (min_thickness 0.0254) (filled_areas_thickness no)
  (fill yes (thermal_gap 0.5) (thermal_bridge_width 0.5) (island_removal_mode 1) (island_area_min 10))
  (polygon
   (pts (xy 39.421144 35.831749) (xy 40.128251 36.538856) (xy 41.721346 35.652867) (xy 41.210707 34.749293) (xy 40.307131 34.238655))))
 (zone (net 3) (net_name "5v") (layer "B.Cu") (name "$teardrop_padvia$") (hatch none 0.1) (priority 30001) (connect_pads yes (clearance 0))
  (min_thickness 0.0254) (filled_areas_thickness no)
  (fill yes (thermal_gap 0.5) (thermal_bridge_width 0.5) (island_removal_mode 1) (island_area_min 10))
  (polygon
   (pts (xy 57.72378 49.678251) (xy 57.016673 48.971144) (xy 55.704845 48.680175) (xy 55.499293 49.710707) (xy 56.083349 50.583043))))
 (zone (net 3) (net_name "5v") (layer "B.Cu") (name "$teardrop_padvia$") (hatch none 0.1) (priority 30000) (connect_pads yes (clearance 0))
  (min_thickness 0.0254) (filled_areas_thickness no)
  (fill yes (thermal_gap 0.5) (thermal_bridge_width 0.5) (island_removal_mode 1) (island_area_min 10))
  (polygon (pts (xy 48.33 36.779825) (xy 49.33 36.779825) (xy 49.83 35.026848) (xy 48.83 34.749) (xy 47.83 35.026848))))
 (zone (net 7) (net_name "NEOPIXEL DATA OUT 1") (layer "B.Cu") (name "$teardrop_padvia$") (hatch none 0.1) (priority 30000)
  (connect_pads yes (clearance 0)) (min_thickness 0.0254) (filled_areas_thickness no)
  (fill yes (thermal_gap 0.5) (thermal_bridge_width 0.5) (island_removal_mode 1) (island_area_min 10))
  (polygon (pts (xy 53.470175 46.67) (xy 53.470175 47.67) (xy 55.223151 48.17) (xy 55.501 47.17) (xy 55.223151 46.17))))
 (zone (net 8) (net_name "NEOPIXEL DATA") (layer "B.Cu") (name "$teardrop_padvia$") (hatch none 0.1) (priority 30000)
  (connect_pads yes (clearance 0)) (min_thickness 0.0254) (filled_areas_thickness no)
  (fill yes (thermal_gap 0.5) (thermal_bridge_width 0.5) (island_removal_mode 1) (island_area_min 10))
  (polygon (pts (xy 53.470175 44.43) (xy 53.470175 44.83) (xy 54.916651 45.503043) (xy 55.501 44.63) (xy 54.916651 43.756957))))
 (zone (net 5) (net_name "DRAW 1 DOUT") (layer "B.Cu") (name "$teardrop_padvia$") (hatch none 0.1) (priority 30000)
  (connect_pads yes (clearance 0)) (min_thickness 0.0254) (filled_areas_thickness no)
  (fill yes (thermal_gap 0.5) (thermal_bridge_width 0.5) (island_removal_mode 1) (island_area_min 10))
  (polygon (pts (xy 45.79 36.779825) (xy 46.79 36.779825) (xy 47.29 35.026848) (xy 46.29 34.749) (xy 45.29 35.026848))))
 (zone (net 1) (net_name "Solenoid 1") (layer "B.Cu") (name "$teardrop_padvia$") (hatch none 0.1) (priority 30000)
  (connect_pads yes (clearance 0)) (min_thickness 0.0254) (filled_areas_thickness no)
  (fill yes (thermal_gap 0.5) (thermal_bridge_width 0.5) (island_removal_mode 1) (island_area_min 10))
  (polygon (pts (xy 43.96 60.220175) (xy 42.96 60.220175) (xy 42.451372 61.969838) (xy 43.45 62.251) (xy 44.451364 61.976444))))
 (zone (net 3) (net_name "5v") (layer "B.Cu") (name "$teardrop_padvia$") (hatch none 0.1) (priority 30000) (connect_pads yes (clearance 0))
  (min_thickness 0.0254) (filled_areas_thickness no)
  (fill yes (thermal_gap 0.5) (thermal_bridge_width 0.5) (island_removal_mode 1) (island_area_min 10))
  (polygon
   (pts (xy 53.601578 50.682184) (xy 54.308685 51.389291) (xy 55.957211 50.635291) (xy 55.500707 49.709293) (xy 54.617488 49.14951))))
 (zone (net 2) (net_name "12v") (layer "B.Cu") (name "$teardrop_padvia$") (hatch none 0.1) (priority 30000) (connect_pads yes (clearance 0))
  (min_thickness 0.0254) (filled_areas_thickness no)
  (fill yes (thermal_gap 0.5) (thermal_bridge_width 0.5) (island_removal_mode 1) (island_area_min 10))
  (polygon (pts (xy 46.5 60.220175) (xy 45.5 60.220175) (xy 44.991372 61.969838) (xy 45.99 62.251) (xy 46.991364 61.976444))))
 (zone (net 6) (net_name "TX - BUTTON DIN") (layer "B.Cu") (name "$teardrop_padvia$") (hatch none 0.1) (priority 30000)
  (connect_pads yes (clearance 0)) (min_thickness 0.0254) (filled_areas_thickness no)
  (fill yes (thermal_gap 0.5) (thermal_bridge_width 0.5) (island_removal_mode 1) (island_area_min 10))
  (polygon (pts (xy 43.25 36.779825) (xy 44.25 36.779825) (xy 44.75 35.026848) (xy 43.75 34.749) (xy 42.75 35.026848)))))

